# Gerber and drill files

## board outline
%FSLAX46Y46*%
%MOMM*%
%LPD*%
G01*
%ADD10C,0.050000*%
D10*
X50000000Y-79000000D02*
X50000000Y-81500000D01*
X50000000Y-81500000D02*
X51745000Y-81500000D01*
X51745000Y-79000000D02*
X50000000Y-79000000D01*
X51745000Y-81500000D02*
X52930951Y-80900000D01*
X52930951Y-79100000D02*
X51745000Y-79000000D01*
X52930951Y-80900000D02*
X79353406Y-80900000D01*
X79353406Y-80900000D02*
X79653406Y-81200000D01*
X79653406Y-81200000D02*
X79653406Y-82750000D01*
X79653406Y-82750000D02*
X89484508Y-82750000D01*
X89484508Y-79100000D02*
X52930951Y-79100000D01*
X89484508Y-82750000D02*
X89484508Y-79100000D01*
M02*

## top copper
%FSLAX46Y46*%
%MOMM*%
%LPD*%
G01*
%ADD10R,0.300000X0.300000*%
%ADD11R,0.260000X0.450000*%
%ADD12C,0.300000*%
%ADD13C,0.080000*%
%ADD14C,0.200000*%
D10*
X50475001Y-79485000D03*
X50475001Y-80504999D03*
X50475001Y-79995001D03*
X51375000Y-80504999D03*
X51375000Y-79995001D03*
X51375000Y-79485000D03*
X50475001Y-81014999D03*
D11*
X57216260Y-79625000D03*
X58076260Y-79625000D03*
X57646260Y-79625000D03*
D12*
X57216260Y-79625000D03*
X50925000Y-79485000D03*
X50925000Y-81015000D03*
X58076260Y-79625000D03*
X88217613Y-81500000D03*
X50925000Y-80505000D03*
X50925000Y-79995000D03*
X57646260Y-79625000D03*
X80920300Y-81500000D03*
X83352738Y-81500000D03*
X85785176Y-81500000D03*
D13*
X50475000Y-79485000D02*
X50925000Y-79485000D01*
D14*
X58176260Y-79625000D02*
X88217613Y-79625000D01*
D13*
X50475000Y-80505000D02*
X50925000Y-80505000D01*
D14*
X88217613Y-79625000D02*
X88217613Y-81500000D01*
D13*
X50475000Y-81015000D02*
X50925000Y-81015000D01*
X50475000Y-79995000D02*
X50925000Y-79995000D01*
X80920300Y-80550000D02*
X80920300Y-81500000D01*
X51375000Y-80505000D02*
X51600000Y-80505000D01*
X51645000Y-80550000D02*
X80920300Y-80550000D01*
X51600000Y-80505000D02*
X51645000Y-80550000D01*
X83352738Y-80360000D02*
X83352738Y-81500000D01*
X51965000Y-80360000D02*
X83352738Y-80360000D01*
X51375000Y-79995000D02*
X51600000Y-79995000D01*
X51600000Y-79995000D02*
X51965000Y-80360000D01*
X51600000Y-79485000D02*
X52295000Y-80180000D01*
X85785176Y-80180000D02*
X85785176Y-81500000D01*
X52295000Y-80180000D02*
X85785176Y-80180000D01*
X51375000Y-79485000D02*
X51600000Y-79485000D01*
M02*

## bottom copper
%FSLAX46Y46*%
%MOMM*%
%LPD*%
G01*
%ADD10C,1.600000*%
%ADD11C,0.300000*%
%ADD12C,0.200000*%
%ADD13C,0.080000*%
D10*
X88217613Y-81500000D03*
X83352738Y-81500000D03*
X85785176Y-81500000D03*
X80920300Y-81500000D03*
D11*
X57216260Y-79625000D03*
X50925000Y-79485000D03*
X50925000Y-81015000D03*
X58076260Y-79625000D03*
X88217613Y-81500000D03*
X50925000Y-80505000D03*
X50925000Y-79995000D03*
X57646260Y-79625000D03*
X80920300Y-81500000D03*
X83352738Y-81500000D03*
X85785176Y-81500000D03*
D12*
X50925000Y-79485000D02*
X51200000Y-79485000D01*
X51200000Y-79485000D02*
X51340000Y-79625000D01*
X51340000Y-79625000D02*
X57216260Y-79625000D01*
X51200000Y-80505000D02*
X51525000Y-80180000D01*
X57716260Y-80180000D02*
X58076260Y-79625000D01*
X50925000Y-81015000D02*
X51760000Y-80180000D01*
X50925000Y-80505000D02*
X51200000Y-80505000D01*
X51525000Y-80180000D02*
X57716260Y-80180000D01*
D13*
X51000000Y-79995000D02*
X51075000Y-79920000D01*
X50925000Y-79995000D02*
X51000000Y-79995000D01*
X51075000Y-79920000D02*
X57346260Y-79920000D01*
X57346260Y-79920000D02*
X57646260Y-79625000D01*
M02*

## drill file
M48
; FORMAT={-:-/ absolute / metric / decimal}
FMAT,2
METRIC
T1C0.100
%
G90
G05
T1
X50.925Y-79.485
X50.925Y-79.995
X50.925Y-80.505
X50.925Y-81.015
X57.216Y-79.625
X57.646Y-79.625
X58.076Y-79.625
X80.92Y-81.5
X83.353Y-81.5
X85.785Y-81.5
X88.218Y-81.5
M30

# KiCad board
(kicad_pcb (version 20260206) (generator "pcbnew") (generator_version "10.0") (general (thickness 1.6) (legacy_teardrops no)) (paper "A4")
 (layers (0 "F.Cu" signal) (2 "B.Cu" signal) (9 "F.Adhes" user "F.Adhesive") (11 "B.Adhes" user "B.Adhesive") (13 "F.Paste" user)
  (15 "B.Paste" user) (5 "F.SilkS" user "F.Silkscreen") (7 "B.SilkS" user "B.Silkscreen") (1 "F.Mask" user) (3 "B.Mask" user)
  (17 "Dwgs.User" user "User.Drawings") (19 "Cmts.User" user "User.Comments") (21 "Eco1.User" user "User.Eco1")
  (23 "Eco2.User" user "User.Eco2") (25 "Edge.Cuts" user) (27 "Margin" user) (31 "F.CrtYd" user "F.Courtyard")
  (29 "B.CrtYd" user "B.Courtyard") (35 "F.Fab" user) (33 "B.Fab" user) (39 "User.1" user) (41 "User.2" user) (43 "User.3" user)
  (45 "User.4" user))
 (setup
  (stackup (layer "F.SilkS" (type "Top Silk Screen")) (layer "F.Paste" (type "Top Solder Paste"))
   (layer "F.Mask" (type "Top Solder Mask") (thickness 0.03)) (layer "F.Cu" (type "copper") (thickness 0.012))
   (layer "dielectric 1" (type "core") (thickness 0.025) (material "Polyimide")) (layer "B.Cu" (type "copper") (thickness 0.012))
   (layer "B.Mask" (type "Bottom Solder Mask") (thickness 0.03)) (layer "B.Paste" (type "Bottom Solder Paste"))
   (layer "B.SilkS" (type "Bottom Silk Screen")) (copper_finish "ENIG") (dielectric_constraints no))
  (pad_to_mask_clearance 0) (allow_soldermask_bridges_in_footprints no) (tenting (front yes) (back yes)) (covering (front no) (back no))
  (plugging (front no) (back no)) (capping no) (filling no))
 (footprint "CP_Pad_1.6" (layer "F.Cu") (at 88.217613 81.5)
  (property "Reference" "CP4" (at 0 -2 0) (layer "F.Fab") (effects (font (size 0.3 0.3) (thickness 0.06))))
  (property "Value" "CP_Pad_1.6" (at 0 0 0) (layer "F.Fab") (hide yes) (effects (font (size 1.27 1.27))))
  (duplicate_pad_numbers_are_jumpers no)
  (pad "1" smd circle (at 0 0) (size 1.6 1.6) (layers "B.Cu" "B.Mask") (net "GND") (solder_mask_margin 0.1)))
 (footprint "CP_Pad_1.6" (layer "F.Cu") (at 83.352738 81.5)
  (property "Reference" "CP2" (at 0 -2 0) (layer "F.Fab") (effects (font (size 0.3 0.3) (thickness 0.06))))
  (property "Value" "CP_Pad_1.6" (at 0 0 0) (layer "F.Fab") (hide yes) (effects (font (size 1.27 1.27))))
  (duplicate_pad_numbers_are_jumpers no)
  (pad "1" smd circle (at 0 0) (size 1.6 1.6) (layers "B.Cu" "B.Mask") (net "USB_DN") (solder_mask_margin 0.1)))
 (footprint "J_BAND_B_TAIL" (layer "F.Cu") (at 50.9 80.25)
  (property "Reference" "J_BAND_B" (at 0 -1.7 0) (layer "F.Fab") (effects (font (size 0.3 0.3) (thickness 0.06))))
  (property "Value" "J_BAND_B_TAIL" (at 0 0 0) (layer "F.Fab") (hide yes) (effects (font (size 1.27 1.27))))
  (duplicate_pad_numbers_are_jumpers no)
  (pad "1" smd rect (at -0.424999 -0.765) (size 0.3 0.3) (layers "F.Cu" "F.Mask") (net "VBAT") (solder_mask_margin 0.05)
   (thermal_bridge_angle 45))
  (pad "2" smd rect (at -0.424999 0.254999) (size 0.3 0.3) (layers "F.Cu" "F.Mask") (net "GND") (solder_mask_margin 0.05)
   (thermal_bridge_angle 45))
  (pad "3" smd rect (at -0.424999 -0.254999) (size 0.3 0.3) (layers "F.Cu" "F.Mask") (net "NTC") (solder_mask_margin 0.05)
   (thermal_bridge_angle 45))
  (pad "4" smd rect (at 0.475 0.254999) (size 0.3 0.3) (layers "F.Cu" "F.Mask") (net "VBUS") (solder_mask_margin 0.05)
   (thermal_bridge_angle 45))
  (pad "5" smd rect (at 0.475 -0.254999) (size 0.3 0.3) (layers "F.Cu" "F.Mask") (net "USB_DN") (solder_mask_margin 0.05)
   (thermal_bridge_angle 45))
  (pad "6" smd rect (at 0.475 -0.765) (size 0.3 0.3) (layers "F.Cu" "F.Mask") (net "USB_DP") (solder_mask_margin 0.05)
   (thermal_bridge_angle 45))
  (pad "7" smd rect (at -0.424999 0.764999) (size 0.3 0.3) (layers "F.Cu" "F.Mask") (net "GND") (solder_mask_margin 0.05)
   (thermal_bridge_angle 45)))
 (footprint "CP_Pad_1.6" (layer "F.Cu") (at 85.785176 81.5)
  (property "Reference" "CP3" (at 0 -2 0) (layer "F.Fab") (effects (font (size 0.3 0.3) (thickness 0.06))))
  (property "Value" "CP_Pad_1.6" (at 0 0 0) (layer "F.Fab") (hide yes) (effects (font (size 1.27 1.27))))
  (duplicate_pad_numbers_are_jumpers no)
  (pad "1" smd circle (at 0 0) (size 1.6 1.6) (layers "B.Cu" "B.Mask") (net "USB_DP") (solder_mask_margin 0.1)))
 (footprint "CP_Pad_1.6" (layer "F.Cu") (at 80.9203 81.5)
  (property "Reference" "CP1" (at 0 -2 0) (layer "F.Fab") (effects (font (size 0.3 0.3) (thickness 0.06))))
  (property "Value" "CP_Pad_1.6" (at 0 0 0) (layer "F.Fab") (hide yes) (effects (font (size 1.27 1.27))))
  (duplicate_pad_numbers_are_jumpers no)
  (pad "1" smd circle (at 0 0) (size 1.6 1.6) (layers "B.Cu" "B.Mask") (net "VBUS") (solder_mask_margin 0.1)))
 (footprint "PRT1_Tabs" (layer "F.Cu") (at 57.64626 79.625)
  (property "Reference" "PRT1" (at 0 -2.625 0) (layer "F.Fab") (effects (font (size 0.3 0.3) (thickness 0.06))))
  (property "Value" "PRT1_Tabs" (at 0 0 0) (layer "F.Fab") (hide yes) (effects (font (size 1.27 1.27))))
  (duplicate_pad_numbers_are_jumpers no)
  (pad "1" smd rect (at -0.43 0) (size 0.26 0.45) (layers "F.Cu" "F.Mask") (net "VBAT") (solder_mask_margin 0.05) (thermal_bridge_angle 45))
  (pad "2" smd rect (at 0.43 0) (size 0.26 0.45) (layers "F.Cu" "F.Mask") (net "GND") (solder_mask_margin 0.05) (thermal_bridge_angle 45))
  (pad "3" smd rect (at 0 0) (size 0.26 0.45) (layers "F.Cu" "F.Mask") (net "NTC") (solder_mask_margin 0.05) (thermal_bridge_angle 45)))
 (gr_line (start 50 79) (end 50 81.5) (stroke (width 0.05) (type default)) (layer "Edge.Cuts"))
 (gr_line (start 50 81.5) (end 51.745 81.5) (stroke (width 0.05) (type default)) (layer "Edge.Cuts"))
 (gr_line (start 51.745 79) (end 50 79) (stroke (width 0.05) (type default)) (layer "Edge.Cuts"))
 (gr_line (start 51.745 81.5) (end 52.930951 80.9) (stroke (width 0.05) (type default)) (layer "Edge.Cuts"))
 (gr_line (start 52.930951 79.1) (end 51.745 79) (stroke (width 0.05) (type default)) (layer "Edge.Cuts"))
 (gr_line (start 52.930951 80.9) (end 79.353406 80.9) (stroke (width 0.05) (type default)) (layer "Edge.Cuts"))
 (gr_line (start 79.353406 80.9) (end 79.653406 81.2) (stroke (width 0.05) (type default)) (layer "Edge.Cuts"))
 (gr_line (start 79.653406 81.2) (end 79.653406 82.75) (stroke (width 0.05) (type default)) (layer "Edge.Cuts"))
 (gr_line (start 79.653406 82.75) (end 89.484508 82.75) (stroke (width 0.05) (type default)) (layer "Edge.Cuts"))
 (gr_line (start 89.484508 79.1) (end 52.930951 79.1) (stroke (width 0.05) (type default)) (layer "Edge.Cuts"))
 (gr_line (start 89.484508 82.75) (end 89.484508 79.1) (stroke (width 0.05) (type default)) (layer "Edge.Cuts"))
 (segment (start 50.475 79.485) (end 50.925 79.485) (width 0.08) (layer "F.Cu") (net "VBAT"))
 (via (at 57.21626 79.625) (size 0.3) (drill 0.1) (layers "F.Cu" "B.Cu") (tenting (front yes) (back yes)) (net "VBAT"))
 (via (at 50.925 79.485) (size 0.3) (drill 0.1) (layers "F.Cu" "B.Cu") (tenting (front yes) (back yes)) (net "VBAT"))
 (segment (start 51.2 79.485) (end 51.34 79.625) (width 0.2) (layer "B.Cu") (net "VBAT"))
 (segment (start 50.925 79.485) (end 51.2 79.485) (width 0.2) (layer "B.Cu") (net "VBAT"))
 (segment (start 51.34 79.625) (end 57.21626 79.625) (width 0.2) (layer "B.Cu") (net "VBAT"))
 (segment (start 88.217613 79.625) (end 88.217613 81.5) (width 0.2) (layer "F.Cu") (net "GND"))
 (segment (start 50.475 80.505) (end 50.925 80.505) (width 0.08) (layer "F.Cu") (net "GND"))
 (segment (start 50.475 81.015) (end 50.925 81.015) (width 0.08) (layer "F.Cu") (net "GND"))
 (segment (start 58.17626 79.625) (end 88.217613 79.625) (width 0.2) (layer "F.Cu") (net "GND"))
 (via (at 50.925 80.505) (size 0.3) (drill 0.1) (layers "F.Cu" "B.Cu") (tenting (front yes) (back yes)) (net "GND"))
 (via (at 50.925 81.015) (size 0.3) (drill 0.1) (layers "F.Cu" "B.Cu") (tenting (front yes) (back yes)) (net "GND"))
 (via (at 58.07626 79.625) (size 0.3) (drill 0.1) (layers "F.Cu" "B.Cu") (tenting (front yes) (back yes)) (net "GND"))
 (via (at 88.217613 81.5) (size 0.3) (drill 0.1) (layers "F.Cu" "B.Cu") (tenting (front yes) (back yes)) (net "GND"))
 (segment (start 51.2 80.505) (end 51.525 80.18) (width 0.2) (layer "B.Cu") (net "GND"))
 (segment (start 50.925 80.505) (end 51.2 80.505) (width 0.2) (layer "B.Cu") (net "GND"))
 (segment (start 50.925 81.015) (end 51.76 80.18) (width 0.2) (layer "B.Cu") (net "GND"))
 (segment (start 57.71626 80.18) (end 58.07626 79.625) (width 0.2) (layer "B.Cu") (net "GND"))
 (segment (start 51.525 80.18) (end 57.71626 80.18) (width 0.2) (layer "B.Cu") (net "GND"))
 (segment (start 50.475 79.995) (end 50.925 79.995) (width 0.08) (layer "F.Cu") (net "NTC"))
 (via (at 50.925 79.995) (size 0.3) (drill 0.1) (layers "F.Cu" "B.Cu") (tenting (front yes) (back yes)) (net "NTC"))
 (via (at 57.64626 79.625) (size 0.3) (drill 0.1) (layers "F.Cu" "B.Cu") (tenting (front yes) (back yes)) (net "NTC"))
 (segment (start 51.075 79.92) (end 57.34626 79.92) (width 0.08) (layer "B.Cu") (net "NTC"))
 (segment (start 57.34626 79.92) (end 57.64626 79.625) (width 0.08) (layer "B.Cu") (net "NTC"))
 (segment (start 50.925 79.995) (end 51 79.995) (width 0.08) (layer "B.Cu") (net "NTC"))
 (segment (start 51 79.995) (end 51.075 79.92) (width 0.08) (layer "B.Cu") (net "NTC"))
 (segment (start 51.645 80.55) (end 80.9203 80.55) (width 0.08) (layer "F.Cu") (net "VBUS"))
 (segment (start 51.6 80.505) (end 51.645 80.55) (width 0.08) (layer "F.Cu") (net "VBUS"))
 (segment (start 80.9203 80.55) (end 80.9203 81.5) (width 0.08) (layer "F.Cu") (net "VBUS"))
 (segment (start 51.375 80.505) (end 51.6 80.505) (width 0.08) (layer "F.Cu") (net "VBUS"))
 (via (at 80.9203 81.5) (size 0.3) (drill 0.1) (layers "F.Cu" "B.Cu") (tenting (front yes) (back yes)) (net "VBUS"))
 (segment (start 51.375 79.995) (end 51.6 79.995) (width 0.08) (layer "F.Cu") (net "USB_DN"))
 (segment (start 83.352738 80.36) (end 83.352738 81.5) (width 0.08) (layer "F.Cu") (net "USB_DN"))
 (segment (start 51.6 79.995) (end 51.965 80.36) (width 0.08) (layer "F.Cu") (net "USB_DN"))
 (segment (start 51.965 80.36) (end 83.352738 80.36) (width 0.08) (layer "F.Cu") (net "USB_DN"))
 (via (at 83.352738 81.5) (size 0.3) (drill 0.1) (layers "F.Cu" "B.Cu") (tenting (front yes) (back yes)) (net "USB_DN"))
 (segment (start 51.375 79.485) (end 51.6 79.485) (width 0.08) (layer "F.Cu") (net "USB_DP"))
 (segment (start 52.295 80.18) (end 85.785176 80.18) (width 0.08) (layer "F.Cu") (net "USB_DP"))
 (segment (start 51.6 79.485) (end 52.295 80.18) (width 0.08) (layer "F.Cu") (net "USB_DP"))
 (segment (start 85.785176 80.18) (end 85.785176 81.5) (width 0.08) (layer "F.Cu") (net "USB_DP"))
 (via (at 85.785176 81.5) (size 0.3) (drill 0.1) (layers "F.Cu" "B.Cu") (tenting (front yes) (back yes)) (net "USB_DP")))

